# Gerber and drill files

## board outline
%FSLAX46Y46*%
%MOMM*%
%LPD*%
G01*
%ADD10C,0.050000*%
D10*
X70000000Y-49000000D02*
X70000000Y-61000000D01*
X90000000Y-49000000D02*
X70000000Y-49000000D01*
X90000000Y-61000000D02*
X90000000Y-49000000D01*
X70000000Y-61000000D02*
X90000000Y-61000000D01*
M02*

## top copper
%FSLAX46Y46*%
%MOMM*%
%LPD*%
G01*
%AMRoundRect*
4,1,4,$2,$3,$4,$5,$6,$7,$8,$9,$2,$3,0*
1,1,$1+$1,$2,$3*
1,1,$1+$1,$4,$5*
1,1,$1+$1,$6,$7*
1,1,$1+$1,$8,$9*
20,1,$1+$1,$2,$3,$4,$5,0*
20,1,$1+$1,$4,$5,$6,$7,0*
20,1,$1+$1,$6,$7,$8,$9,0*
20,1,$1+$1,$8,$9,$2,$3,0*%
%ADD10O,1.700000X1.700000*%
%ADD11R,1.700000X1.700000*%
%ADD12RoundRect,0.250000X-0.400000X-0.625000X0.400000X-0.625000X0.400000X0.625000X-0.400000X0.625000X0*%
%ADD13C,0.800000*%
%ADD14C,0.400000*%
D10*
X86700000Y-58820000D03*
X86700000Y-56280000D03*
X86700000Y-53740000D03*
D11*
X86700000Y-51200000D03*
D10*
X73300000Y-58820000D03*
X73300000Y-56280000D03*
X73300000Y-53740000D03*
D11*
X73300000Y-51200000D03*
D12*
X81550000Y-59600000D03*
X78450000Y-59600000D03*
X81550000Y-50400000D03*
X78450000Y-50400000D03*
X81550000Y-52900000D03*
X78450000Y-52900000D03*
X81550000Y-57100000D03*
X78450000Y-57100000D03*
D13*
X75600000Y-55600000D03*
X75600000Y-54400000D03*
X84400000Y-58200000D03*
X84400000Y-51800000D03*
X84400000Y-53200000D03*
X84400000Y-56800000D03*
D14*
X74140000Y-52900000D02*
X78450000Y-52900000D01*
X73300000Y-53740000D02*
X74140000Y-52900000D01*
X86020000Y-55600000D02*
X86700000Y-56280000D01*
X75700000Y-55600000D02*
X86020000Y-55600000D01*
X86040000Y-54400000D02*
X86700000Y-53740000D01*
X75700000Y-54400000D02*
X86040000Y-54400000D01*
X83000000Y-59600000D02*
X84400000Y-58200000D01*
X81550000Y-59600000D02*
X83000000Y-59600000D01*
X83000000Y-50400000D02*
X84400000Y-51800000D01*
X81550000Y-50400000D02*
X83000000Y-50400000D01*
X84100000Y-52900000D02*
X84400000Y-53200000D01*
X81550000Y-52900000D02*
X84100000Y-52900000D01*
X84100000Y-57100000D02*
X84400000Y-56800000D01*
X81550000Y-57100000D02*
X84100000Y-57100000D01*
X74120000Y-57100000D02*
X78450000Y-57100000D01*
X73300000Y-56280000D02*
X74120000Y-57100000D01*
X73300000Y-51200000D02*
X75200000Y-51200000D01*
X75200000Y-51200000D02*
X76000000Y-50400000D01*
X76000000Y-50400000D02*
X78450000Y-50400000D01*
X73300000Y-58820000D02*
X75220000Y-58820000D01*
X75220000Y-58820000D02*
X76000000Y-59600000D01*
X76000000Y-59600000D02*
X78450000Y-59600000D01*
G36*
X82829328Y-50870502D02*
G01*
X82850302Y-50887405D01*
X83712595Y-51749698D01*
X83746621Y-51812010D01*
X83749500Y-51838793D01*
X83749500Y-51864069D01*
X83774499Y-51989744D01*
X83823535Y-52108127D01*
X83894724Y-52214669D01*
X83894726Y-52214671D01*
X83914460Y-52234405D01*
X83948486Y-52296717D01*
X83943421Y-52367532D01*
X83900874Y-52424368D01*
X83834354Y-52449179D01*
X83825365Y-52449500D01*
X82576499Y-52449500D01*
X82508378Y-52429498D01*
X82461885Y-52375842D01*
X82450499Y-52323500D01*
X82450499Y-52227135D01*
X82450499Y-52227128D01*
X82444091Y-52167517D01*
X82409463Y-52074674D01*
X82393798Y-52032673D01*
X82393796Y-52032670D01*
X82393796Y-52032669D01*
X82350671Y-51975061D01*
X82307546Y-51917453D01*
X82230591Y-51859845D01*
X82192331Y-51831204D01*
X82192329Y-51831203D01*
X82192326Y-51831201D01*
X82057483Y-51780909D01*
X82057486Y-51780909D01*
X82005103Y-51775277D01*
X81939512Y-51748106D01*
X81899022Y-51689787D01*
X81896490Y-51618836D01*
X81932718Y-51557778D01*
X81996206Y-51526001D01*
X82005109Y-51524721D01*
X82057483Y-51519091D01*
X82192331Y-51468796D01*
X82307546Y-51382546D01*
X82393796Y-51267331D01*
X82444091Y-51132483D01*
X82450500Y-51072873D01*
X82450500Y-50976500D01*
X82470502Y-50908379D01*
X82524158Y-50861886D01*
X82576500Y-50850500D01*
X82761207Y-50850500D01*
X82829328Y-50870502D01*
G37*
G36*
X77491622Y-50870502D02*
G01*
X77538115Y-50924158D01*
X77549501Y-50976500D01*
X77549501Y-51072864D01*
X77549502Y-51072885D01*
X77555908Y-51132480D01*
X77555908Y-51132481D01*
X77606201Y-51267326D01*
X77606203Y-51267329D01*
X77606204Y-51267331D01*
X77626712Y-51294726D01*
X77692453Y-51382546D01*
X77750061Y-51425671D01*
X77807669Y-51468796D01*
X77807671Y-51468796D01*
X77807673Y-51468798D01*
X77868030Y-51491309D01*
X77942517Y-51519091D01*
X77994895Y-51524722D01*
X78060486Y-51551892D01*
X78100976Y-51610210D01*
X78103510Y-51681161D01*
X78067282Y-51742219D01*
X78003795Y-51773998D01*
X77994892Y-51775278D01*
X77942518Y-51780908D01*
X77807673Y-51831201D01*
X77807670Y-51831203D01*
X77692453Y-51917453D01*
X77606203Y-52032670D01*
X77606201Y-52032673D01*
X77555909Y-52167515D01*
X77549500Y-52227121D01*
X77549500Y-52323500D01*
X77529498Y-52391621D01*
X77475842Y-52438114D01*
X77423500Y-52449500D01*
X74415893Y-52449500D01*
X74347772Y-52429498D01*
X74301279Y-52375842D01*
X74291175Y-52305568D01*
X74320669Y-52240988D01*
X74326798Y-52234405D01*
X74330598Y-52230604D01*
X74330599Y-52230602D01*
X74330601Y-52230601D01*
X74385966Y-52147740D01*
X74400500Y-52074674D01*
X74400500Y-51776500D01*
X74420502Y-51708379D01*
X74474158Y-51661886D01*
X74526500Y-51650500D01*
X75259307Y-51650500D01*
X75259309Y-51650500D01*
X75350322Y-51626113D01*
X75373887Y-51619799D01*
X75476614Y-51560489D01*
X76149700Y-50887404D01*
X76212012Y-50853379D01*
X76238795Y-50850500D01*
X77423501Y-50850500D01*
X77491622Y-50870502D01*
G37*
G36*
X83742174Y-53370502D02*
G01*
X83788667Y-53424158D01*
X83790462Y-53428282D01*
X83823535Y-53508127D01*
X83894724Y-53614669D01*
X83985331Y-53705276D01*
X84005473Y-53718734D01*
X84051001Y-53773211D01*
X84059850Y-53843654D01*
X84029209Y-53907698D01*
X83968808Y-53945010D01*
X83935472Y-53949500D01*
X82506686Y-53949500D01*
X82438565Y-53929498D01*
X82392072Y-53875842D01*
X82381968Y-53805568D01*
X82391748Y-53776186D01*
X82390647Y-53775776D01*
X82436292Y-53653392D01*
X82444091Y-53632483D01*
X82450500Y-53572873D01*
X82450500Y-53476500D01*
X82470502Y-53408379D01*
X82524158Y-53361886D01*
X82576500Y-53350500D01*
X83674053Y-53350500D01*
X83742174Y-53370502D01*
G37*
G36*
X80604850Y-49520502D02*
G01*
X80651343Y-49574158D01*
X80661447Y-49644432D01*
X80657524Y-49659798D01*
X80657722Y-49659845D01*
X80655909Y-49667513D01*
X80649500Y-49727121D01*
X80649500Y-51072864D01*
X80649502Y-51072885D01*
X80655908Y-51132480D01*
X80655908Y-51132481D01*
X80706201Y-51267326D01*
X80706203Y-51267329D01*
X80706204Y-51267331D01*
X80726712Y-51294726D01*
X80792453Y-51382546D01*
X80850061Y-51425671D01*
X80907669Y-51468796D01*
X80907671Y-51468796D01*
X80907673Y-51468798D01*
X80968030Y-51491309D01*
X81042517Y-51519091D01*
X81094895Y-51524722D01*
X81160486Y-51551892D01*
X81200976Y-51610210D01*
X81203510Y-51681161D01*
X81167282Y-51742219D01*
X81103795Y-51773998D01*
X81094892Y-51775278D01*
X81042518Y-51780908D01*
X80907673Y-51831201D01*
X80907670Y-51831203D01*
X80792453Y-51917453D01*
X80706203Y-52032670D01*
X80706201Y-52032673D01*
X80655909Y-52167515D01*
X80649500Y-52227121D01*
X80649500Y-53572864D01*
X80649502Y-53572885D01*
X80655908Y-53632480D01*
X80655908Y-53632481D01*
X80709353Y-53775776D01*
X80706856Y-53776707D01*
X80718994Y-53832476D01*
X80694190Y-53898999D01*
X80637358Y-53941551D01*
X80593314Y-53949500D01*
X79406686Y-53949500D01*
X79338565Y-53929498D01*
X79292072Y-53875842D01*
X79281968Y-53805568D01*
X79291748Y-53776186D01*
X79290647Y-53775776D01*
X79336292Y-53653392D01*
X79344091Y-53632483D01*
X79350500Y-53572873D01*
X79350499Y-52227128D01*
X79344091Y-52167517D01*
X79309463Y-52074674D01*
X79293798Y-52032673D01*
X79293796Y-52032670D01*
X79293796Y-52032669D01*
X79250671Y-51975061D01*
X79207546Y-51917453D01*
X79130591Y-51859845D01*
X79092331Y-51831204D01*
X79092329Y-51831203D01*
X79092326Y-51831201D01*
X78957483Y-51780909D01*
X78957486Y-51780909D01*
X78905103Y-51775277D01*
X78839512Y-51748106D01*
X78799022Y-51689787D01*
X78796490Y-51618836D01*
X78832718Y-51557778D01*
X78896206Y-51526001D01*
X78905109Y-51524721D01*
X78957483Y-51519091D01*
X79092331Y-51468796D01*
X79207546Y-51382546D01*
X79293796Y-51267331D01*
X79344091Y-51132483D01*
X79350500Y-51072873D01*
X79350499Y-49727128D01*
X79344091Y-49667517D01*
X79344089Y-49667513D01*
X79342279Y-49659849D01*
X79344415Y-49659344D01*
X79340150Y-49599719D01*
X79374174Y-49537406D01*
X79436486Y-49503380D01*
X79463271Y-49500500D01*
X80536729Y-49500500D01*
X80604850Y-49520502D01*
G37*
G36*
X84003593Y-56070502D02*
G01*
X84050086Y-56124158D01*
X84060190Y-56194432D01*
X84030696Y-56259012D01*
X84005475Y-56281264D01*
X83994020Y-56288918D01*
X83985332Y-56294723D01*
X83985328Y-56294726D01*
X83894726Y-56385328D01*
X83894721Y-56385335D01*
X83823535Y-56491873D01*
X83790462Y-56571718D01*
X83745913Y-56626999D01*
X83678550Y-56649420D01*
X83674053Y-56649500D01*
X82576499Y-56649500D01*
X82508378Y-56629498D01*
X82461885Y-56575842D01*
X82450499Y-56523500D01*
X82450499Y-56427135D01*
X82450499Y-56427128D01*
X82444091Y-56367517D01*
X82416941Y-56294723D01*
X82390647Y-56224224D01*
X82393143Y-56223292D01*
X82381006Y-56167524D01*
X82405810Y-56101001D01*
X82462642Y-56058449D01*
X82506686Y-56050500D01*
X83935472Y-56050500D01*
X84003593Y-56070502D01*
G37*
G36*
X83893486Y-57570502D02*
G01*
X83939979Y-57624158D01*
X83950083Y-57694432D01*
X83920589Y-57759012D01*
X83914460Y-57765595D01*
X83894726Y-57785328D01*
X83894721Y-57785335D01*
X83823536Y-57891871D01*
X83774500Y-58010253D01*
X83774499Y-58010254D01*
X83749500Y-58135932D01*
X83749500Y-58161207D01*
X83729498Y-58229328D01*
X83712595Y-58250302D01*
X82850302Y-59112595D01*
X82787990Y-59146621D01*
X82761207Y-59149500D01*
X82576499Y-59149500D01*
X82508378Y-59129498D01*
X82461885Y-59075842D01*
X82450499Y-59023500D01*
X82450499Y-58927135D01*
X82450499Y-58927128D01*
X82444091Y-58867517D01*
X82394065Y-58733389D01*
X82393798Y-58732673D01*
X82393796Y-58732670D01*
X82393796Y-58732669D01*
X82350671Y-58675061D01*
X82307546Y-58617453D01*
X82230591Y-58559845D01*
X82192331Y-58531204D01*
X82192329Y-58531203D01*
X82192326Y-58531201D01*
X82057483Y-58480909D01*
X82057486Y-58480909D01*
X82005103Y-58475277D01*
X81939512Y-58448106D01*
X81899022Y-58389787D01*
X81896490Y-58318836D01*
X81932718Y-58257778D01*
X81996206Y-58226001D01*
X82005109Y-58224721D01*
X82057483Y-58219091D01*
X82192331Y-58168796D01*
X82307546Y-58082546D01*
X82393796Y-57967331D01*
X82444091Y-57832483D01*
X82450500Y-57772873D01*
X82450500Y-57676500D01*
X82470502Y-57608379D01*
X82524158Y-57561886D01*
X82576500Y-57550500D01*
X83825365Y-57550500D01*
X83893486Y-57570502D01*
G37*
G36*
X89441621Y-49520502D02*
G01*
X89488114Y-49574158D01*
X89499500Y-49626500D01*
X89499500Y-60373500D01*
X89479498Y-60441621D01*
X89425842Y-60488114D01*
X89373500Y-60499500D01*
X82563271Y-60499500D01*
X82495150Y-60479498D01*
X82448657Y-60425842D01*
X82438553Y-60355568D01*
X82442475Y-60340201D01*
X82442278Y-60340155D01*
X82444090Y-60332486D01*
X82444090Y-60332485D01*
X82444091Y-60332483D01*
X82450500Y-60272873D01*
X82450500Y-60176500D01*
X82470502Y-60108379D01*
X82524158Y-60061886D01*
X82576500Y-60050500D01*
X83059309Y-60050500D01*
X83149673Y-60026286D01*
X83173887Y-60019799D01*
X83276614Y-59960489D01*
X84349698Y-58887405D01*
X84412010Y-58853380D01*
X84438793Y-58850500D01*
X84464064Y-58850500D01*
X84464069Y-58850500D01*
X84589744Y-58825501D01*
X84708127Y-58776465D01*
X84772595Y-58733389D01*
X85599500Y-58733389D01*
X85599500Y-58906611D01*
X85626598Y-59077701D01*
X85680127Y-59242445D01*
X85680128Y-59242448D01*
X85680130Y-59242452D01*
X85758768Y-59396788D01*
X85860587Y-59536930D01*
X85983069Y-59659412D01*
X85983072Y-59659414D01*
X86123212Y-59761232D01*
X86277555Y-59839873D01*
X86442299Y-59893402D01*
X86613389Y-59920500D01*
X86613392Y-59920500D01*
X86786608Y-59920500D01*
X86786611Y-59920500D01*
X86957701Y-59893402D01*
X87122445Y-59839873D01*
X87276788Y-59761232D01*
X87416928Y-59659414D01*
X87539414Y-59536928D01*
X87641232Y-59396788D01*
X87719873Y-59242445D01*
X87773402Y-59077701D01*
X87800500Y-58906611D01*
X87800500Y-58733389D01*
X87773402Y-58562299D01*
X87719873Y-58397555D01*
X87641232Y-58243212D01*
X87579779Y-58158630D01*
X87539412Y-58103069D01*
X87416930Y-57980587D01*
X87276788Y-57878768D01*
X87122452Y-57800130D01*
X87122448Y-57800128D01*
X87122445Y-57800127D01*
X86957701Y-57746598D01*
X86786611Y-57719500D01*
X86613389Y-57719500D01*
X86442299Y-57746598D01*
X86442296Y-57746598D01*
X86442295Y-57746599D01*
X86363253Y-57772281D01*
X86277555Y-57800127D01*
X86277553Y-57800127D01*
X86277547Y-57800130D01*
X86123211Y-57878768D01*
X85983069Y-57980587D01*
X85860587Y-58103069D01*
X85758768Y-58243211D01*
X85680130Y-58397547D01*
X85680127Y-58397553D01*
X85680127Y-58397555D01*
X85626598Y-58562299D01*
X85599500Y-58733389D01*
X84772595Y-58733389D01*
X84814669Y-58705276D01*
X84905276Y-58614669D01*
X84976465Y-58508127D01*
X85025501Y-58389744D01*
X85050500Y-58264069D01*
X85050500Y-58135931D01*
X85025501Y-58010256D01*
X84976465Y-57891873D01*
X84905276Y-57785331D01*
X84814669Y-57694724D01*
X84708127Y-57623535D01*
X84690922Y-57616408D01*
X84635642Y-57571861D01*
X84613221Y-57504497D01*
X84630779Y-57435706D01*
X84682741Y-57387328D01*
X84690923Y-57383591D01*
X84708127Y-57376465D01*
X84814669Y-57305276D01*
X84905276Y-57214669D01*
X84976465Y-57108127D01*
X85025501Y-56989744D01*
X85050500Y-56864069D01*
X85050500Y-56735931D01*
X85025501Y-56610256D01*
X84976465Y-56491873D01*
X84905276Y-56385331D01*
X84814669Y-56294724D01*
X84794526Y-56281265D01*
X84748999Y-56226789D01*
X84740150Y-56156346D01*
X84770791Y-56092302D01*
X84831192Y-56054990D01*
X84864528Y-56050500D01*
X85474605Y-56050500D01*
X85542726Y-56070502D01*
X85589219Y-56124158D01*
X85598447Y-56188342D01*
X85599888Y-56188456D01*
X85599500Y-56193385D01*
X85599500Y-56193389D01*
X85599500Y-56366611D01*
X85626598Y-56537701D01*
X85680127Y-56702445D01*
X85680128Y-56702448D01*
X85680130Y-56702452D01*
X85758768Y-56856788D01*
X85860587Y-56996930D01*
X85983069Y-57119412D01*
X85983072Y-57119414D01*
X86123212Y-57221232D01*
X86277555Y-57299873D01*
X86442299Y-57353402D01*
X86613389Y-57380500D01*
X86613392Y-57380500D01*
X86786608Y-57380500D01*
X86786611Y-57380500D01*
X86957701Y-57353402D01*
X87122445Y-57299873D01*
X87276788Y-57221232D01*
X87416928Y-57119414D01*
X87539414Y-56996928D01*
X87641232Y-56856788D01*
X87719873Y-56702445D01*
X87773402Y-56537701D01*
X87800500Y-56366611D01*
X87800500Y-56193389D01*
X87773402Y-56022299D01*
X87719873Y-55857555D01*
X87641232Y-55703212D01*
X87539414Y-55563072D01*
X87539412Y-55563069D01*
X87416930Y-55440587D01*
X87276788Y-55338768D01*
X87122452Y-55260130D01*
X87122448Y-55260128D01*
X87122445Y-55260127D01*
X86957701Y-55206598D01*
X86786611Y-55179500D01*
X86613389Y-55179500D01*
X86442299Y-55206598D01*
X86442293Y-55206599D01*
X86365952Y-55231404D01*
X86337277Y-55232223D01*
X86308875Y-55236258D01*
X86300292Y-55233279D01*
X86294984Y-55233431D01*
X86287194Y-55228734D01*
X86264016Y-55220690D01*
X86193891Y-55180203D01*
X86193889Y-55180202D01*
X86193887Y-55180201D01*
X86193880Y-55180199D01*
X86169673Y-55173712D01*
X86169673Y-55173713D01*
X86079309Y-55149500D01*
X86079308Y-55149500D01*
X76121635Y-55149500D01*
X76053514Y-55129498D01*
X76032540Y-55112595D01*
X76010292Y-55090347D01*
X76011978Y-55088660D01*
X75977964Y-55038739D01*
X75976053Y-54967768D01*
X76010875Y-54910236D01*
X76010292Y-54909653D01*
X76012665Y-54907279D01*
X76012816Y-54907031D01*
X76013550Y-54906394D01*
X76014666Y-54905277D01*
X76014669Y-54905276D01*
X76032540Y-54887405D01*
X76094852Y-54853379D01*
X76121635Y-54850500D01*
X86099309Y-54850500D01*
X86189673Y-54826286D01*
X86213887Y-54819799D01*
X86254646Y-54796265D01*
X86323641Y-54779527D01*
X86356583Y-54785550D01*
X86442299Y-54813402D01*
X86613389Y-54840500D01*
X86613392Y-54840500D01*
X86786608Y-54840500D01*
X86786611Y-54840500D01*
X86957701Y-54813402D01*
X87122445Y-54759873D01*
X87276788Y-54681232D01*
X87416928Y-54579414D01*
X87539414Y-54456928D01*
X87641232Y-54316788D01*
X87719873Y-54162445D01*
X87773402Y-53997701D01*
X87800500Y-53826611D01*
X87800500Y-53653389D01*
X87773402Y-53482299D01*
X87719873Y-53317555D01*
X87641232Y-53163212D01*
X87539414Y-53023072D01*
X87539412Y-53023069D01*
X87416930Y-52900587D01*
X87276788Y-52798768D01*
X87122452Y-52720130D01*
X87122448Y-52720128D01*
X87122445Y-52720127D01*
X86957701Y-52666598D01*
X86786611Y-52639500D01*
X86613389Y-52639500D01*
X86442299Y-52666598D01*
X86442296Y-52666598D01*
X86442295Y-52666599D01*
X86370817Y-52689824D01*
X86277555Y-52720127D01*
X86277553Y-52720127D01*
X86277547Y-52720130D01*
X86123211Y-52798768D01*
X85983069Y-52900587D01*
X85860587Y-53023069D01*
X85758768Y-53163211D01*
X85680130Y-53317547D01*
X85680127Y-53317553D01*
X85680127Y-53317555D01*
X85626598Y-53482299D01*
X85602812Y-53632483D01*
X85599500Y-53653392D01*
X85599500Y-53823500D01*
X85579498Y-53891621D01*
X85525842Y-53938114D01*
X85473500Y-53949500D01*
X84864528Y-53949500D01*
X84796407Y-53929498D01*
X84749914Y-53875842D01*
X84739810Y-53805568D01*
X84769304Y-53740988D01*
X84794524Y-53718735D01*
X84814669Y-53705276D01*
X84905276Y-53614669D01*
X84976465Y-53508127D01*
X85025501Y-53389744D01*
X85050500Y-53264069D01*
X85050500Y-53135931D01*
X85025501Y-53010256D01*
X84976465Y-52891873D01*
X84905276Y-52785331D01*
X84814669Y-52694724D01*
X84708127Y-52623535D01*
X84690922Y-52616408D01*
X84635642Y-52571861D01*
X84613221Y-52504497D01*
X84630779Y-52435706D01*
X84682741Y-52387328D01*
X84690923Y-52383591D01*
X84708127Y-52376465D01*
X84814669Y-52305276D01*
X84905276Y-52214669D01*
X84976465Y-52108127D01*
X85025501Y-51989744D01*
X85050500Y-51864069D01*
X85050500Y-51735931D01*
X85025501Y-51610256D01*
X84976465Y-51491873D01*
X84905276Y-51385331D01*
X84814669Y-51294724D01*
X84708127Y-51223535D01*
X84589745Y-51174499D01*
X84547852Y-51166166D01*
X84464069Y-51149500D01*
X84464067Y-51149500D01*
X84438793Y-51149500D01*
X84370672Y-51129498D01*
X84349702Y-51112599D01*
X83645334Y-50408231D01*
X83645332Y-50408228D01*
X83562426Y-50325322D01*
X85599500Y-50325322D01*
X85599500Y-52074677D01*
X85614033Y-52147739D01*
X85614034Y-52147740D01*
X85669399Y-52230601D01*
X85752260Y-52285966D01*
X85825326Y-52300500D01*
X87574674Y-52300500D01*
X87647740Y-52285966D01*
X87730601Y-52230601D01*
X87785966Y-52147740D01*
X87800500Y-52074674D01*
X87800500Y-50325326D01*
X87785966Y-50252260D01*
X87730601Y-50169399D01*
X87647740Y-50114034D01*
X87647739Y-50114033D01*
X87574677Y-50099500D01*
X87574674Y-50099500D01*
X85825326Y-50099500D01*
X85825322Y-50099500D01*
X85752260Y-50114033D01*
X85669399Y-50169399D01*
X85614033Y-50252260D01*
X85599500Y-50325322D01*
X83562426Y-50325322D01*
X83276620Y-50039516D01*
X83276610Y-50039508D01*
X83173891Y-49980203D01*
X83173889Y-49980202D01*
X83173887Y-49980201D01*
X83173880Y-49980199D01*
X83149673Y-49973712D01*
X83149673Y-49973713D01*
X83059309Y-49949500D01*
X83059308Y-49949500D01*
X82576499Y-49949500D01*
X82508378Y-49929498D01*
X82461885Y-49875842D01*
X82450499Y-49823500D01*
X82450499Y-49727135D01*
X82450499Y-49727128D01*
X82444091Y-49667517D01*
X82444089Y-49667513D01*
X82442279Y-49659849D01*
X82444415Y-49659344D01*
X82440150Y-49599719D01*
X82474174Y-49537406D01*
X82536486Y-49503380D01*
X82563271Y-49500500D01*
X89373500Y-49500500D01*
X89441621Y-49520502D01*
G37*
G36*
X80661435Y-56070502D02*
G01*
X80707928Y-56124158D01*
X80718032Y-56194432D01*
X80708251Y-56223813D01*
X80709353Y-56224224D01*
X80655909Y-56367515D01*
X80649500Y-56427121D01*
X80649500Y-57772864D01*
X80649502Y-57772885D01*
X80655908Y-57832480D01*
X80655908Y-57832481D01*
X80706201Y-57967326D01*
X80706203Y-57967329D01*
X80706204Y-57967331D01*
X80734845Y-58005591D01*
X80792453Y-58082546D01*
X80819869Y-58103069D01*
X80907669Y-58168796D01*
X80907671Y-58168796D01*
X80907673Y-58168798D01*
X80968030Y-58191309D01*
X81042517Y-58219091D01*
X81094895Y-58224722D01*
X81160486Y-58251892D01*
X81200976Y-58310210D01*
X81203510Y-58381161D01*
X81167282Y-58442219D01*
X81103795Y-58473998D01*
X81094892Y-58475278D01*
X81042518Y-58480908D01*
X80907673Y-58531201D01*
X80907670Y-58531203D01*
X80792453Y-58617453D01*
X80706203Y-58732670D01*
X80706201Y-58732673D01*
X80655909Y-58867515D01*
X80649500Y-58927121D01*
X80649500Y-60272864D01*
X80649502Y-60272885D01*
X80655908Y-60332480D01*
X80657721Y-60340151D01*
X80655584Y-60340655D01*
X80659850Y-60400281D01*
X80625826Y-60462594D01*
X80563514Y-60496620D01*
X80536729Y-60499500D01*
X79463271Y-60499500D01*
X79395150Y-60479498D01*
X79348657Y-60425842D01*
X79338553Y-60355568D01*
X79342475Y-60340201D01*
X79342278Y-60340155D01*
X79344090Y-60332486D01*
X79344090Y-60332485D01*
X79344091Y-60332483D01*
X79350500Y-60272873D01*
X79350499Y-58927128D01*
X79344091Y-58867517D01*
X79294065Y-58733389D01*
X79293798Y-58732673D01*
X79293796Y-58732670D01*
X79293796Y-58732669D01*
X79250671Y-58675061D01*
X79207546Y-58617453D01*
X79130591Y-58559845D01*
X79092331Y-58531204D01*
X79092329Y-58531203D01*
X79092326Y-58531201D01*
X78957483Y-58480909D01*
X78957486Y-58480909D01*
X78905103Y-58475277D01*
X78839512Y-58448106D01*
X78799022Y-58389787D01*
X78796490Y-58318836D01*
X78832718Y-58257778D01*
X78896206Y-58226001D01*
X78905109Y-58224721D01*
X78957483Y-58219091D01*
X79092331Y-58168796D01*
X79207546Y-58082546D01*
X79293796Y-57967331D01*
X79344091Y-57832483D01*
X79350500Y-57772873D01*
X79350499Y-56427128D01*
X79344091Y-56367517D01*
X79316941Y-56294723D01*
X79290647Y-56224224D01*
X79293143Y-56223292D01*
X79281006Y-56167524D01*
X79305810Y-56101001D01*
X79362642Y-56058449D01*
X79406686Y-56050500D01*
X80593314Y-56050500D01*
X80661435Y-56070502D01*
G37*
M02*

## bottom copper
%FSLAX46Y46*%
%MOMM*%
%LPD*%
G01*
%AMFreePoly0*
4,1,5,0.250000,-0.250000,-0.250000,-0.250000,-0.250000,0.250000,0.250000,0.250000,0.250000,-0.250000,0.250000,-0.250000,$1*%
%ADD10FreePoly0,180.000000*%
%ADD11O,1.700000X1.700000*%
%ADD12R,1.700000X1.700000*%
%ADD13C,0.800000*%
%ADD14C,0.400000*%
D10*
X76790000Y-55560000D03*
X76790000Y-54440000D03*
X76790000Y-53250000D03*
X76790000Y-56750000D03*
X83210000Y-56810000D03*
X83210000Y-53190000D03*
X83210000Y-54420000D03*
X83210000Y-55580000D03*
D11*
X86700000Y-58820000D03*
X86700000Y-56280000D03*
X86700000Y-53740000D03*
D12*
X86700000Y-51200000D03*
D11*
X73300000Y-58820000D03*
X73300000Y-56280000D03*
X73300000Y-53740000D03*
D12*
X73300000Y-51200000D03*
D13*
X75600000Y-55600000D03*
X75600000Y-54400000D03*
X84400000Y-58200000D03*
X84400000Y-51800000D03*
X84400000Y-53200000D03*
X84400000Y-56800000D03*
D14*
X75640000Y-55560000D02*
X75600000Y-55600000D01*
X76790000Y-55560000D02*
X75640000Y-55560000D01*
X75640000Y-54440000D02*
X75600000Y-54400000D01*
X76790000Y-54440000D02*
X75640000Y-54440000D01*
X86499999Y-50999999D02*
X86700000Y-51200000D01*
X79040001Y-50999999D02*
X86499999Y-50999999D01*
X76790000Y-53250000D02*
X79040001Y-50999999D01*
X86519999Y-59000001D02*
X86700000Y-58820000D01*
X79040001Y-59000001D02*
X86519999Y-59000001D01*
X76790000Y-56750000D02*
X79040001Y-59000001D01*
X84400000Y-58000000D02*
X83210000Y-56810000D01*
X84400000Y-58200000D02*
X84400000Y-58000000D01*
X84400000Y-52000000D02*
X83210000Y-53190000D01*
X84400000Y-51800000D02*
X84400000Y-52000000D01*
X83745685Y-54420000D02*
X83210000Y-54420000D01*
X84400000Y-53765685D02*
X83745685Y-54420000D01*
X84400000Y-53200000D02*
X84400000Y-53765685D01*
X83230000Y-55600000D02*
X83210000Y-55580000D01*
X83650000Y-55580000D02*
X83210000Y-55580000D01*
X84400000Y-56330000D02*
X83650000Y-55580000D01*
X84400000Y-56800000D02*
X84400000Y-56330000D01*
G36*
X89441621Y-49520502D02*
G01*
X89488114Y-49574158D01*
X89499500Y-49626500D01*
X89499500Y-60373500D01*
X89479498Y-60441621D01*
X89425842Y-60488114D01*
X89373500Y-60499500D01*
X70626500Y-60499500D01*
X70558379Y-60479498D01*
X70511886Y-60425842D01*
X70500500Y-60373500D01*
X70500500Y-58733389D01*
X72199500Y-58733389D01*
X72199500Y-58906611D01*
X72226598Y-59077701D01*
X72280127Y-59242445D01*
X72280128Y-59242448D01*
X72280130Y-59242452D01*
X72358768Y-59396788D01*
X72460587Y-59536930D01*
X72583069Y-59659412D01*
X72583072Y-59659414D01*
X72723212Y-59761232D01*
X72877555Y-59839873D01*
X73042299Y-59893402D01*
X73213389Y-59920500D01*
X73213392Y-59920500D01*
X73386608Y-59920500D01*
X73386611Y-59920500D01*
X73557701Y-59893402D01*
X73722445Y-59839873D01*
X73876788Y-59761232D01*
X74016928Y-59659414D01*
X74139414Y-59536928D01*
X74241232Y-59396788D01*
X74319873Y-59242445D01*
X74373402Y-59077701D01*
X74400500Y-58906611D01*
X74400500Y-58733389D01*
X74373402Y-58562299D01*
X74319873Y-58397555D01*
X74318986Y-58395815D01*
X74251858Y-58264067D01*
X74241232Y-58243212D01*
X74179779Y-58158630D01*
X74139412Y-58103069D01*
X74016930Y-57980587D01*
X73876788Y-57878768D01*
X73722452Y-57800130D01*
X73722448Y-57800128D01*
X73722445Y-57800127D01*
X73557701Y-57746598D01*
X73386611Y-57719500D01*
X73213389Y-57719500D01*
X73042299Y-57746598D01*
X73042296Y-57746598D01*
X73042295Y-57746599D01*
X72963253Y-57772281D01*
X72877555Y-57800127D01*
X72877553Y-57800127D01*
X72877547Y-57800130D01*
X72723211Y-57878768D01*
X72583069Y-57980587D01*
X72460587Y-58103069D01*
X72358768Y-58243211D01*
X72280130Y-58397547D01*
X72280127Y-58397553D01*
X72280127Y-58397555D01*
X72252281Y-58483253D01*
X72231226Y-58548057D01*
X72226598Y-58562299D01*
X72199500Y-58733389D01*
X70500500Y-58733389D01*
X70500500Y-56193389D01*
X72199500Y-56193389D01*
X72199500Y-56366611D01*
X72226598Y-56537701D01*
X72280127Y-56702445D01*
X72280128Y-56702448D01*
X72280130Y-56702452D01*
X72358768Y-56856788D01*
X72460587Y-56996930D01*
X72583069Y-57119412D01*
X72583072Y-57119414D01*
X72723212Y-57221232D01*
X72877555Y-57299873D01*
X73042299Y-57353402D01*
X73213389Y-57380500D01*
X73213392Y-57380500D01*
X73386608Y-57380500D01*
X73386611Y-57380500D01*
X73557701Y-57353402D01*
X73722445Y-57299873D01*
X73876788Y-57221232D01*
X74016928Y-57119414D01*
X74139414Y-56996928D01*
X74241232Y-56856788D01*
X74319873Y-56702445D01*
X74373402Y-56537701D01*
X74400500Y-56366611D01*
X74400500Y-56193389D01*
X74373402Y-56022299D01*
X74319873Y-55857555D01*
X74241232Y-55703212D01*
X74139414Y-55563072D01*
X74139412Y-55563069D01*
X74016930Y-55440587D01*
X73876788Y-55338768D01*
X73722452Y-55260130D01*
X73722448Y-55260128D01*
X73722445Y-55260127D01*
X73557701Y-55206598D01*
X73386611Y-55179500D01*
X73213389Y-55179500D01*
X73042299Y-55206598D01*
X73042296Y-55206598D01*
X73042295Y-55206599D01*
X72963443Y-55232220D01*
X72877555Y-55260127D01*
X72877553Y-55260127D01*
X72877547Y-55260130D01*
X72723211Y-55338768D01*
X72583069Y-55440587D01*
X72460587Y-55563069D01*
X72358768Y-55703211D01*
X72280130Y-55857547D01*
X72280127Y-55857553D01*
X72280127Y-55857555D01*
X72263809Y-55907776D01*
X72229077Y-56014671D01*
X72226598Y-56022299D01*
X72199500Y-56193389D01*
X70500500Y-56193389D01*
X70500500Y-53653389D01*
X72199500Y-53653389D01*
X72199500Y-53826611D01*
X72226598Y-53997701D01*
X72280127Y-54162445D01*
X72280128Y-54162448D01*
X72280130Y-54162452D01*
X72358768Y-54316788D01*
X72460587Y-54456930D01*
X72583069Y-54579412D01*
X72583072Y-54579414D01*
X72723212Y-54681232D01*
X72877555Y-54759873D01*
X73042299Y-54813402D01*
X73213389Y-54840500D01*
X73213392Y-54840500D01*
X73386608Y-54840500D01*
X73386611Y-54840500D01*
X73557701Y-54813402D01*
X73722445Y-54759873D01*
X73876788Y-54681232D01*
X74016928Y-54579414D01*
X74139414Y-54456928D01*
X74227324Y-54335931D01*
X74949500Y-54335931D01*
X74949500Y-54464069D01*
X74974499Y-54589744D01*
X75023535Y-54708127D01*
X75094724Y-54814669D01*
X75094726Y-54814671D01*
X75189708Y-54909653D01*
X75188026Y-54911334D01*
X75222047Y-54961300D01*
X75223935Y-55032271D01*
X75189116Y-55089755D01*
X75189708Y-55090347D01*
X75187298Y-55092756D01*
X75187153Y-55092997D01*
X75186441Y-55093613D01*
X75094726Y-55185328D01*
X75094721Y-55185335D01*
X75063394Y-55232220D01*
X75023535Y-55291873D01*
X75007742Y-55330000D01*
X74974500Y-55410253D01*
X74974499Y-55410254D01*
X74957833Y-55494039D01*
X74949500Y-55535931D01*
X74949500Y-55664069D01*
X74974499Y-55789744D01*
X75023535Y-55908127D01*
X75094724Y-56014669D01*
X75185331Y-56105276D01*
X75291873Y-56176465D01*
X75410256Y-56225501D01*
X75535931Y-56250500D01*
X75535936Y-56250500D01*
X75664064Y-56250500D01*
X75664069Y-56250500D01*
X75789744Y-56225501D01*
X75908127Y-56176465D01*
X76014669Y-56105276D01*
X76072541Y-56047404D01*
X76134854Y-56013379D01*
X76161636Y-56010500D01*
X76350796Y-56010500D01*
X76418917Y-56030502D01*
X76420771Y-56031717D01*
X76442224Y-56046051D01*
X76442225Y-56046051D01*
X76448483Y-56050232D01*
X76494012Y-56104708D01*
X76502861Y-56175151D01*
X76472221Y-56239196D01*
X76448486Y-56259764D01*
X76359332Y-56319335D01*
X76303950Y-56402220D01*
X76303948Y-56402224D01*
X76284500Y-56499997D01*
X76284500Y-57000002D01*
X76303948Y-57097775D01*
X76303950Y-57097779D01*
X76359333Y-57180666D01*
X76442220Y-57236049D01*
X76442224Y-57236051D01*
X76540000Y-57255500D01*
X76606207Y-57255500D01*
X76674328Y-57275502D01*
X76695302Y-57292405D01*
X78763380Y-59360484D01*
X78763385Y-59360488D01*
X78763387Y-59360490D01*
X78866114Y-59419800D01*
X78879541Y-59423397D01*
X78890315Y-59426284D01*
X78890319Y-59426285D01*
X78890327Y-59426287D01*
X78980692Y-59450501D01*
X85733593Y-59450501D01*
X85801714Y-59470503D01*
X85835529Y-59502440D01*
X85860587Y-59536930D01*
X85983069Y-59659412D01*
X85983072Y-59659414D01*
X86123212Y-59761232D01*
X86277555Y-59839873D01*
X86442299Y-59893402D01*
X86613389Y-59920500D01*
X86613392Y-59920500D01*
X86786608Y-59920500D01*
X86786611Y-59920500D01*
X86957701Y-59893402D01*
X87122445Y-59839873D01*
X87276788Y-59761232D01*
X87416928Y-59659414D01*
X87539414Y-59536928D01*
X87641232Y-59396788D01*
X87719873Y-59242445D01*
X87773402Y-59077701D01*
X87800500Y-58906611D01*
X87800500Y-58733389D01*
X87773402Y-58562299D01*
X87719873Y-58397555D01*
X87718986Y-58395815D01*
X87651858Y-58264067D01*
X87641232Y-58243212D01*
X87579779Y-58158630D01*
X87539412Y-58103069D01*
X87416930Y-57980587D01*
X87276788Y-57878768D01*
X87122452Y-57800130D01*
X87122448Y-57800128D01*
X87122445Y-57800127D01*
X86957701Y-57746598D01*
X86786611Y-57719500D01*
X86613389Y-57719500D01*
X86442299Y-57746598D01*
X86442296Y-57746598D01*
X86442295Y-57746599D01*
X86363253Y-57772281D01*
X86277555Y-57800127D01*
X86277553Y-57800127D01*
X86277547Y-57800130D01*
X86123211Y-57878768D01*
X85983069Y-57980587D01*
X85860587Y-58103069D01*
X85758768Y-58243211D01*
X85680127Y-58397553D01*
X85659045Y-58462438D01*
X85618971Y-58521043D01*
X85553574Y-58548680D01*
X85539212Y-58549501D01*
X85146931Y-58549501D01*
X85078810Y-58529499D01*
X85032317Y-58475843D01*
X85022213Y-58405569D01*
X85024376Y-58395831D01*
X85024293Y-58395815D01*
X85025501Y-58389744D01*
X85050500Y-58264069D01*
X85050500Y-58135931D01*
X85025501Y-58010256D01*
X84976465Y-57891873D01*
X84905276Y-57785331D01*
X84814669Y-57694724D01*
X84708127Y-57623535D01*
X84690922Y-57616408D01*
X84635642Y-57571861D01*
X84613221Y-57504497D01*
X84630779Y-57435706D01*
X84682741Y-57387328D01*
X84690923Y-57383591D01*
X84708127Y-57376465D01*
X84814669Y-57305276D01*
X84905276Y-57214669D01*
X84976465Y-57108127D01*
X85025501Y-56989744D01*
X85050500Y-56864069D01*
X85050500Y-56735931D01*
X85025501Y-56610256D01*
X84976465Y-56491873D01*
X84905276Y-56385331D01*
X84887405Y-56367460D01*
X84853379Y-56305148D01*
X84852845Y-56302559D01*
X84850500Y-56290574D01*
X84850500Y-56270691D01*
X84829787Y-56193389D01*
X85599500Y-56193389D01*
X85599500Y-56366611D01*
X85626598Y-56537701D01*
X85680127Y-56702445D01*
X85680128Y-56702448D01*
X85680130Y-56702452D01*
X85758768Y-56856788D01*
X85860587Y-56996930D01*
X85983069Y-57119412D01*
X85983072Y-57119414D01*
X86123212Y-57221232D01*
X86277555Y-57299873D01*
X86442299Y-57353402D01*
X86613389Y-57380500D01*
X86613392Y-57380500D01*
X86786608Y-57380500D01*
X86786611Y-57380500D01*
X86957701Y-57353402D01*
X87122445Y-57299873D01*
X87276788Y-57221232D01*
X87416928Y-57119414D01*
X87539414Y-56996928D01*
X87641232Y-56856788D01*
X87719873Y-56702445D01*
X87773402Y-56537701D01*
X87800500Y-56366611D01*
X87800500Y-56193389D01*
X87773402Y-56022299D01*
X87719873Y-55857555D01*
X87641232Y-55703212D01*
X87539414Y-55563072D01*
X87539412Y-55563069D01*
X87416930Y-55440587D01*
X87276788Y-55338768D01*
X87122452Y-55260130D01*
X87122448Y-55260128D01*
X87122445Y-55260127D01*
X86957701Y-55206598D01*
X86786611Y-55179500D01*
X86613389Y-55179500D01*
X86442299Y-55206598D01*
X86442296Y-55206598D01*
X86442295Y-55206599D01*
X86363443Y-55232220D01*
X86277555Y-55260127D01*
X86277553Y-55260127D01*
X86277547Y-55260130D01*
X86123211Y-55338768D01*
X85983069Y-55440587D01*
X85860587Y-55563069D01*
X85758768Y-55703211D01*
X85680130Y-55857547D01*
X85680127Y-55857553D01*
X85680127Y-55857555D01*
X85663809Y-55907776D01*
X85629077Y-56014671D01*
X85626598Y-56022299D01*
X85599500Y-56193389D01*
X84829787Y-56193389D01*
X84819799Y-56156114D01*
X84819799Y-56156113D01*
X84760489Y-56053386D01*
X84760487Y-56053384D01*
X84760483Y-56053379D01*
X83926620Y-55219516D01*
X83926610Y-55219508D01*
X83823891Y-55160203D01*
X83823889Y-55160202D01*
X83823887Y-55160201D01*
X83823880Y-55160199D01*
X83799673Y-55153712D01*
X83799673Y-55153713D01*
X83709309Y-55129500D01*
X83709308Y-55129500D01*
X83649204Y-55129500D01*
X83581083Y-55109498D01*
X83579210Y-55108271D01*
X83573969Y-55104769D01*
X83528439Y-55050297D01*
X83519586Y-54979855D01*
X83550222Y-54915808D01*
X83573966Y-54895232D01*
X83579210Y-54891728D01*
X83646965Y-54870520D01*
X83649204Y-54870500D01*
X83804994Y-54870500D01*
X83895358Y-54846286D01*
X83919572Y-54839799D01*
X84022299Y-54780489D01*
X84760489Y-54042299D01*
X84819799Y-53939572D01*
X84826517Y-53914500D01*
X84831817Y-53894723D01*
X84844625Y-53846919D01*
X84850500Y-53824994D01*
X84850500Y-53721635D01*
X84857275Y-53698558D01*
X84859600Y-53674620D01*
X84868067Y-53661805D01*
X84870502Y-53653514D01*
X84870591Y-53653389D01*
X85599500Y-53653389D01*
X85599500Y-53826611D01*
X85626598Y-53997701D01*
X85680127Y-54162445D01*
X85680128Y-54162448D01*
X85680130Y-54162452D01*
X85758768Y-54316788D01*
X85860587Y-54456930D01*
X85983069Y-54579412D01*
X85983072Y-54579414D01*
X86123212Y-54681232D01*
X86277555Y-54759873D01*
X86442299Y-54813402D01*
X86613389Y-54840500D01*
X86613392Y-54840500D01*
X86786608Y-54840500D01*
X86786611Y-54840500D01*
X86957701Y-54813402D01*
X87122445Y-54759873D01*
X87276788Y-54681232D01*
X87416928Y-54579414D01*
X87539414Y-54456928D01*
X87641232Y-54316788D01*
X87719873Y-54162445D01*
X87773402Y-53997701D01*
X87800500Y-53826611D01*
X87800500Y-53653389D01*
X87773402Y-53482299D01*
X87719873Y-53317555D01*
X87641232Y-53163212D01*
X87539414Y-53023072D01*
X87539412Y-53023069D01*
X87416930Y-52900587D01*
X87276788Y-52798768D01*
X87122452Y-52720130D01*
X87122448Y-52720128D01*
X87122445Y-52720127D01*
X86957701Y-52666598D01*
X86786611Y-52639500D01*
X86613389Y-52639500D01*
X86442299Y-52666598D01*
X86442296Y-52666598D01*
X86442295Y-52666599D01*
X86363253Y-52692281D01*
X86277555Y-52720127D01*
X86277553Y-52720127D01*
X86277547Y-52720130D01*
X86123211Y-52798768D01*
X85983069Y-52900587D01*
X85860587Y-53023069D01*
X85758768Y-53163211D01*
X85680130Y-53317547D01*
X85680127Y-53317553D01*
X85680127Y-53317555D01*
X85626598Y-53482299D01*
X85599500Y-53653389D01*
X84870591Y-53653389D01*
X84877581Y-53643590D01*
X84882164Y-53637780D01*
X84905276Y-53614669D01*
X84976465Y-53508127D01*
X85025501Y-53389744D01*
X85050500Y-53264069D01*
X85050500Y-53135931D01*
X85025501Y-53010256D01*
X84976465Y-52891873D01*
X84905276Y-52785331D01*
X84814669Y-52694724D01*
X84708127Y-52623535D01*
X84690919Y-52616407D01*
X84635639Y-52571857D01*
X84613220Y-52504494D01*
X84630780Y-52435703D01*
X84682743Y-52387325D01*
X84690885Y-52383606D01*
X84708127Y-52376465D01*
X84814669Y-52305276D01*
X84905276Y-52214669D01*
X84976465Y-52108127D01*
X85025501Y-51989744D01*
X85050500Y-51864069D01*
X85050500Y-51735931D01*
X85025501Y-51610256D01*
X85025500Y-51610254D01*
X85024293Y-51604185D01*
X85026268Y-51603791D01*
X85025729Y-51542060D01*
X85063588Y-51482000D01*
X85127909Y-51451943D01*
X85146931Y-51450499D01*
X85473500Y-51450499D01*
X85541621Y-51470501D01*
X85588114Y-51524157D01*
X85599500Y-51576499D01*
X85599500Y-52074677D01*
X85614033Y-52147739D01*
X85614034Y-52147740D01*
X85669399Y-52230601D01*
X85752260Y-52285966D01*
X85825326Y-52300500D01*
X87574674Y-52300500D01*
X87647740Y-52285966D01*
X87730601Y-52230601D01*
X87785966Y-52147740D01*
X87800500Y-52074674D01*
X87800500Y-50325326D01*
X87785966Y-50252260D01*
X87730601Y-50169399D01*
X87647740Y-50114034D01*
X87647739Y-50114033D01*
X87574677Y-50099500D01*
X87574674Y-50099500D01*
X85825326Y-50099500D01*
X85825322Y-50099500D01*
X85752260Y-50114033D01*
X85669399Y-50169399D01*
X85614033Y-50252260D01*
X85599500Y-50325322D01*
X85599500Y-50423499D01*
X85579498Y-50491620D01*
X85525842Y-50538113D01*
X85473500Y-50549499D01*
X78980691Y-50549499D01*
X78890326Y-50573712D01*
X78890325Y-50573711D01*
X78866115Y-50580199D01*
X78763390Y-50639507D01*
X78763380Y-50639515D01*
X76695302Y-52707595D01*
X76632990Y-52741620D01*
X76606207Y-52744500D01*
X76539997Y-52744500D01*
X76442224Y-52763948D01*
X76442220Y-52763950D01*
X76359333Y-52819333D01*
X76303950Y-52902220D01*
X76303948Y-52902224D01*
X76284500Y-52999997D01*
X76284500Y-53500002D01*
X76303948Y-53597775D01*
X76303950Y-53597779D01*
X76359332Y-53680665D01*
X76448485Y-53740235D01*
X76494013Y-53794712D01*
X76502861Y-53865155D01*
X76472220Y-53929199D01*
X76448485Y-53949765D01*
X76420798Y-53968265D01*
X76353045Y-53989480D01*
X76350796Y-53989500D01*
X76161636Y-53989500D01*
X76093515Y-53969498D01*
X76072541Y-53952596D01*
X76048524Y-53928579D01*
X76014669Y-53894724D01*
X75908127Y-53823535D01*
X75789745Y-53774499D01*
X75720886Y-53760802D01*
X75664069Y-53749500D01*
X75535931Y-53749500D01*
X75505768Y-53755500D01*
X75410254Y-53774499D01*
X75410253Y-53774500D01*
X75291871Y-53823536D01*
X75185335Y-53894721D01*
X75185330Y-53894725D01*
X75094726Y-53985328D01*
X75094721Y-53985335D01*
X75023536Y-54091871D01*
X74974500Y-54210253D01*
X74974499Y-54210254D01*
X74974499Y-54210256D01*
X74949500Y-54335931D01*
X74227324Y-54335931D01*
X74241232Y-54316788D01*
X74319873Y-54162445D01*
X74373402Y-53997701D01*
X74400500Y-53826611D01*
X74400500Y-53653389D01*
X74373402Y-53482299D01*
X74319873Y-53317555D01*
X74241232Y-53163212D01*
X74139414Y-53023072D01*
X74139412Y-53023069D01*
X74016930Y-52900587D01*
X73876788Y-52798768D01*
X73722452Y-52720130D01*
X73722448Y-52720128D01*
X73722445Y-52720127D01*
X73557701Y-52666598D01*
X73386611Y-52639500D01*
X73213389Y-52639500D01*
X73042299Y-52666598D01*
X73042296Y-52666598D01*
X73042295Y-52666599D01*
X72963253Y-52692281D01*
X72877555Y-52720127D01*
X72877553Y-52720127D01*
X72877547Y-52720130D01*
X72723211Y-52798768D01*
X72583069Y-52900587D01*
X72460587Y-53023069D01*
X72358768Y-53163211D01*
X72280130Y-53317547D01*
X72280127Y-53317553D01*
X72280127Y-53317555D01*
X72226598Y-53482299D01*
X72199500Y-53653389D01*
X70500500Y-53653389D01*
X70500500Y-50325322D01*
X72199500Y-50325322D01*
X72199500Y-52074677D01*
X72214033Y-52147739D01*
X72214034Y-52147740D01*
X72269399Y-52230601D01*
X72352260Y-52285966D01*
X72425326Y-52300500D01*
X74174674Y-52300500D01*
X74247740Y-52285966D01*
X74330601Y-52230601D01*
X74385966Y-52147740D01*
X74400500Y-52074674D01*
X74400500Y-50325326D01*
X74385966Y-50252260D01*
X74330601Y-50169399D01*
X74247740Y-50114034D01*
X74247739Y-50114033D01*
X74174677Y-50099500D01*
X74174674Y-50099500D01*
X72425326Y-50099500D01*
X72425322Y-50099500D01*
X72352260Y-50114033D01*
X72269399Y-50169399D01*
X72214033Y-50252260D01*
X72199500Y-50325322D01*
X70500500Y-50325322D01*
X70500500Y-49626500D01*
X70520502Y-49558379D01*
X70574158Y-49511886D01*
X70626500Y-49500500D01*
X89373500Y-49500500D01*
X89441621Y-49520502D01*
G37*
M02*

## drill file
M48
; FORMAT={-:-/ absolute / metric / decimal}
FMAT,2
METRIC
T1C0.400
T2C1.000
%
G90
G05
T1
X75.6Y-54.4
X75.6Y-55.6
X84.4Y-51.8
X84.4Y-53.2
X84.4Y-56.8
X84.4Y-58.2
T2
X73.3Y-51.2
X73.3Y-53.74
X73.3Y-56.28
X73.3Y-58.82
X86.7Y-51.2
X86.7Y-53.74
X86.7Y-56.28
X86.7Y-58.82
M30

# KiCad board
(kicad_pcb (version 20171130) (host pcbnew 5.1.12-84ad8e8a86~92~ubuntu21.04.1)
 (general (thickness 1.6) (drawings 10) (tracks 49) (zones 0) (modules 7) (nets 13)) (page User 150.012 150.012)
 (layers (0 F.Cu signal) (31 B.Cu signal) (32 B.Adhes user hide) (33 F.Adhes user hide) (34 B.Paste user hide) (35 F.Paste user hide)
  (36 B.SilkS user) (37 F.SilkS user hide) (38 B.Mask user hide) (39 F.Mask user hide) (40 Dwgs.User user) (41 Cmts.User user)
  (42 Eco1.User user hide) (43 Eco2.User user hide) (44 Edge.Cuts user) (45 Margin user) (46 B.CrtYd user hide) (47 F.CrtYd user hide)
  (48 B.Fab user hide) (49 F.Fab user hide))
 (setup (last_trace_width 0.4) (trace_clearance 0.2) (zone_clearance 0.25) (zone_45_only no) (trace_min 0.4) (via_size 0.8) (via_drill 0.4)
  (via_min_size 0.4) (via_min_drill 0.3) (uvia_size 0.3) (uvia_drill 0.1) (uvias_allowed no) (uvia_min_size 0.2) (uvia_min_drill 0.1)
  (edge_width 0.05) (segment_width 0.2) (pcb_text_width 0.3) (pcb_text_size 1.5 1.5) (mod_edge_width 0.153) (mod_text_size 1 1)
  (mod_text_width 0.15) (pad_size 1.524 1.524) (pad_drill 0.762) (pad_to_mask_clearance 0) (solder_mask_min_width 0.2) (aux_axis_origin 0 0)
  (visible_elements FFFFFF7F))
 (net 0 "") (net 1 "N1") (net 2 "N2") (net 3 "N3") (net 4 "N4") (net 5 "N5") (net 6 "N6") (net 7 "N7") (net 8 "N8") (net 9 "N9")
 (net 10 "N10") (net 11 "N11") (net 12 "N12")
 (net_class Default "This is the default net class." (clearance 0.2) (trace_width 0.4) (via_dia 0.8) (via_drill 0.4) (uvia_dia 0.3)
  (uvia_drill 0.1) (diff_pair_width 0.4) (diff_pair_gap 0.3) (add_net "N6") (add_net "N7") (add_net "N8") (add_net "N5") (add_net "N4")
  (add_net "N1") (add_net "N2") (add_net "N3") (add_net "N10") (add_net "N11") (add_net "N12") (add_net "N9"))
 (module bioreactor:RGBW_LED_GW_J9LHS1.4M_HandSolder (layer B.Cu) (at 80 55 180)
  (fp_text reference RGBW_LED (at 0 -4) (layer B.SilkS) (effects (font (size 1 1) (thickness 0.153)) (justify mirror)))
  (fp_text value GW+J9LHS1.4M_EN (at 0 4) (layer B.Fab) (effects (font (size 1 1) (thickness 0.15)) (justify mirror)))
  (pad 6 smd custom (at 3.21 -0.56 180) (size 0.5 0.5) (layers B.Cu B.Paste B.Mask) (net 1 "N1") (zone_connect 0)
   (options (clearance outline) (anchor rect)) (primitives))
  (pad 7 smd custom (at 3.21 0.56 180) (size 0.5 0.5) (layers B.Cu B.Paste B.Mask) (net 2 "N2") (zone_connect 0)
   (options (clearance outline) (anchor rect)) (primitives))
  (pad 8 smd custom (at 3.21 1.75 180) (size 0.5 0.5) (layers B.Cu B.Paste B.Mask) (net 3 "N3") (zone_connect 0)
   (options (clearance outline) (anchor rect)) (primitives))
  (pad 5 smd custom (at 3.21 -1.75 180) (size 0.5 0.5) (layers B.Cu B.Paste B.Mask) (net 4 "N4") (zone_connect 0)
   (options (clearance outline) (anchor rect)) (primitives))
  (pad 4 smd custom (at -3.21 -1.81 180) (size 0.5 0.5) (layers B.Cu B.Paste B.Mask) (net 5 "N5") (zone_connect 0)
   (options (clearance outline) (anchor rect)) (primitives))
  (pad 1 smd custom (at -3.21 1.81 180) (size 0.5 0.5) (layers B.Cu B.Paste B.Mask) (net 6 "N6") (zone_connect 0)
   (options (clearance outline) (anchor rect)) (primitives))
  (pad 2 smd custom (at -3.21 0.58 180) (size 0.5 0.5) (layers B.Cu B.Paste B.Mask) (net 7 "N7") (zone_connect 0)
   (options (clearance outline) (anchor rect)) (primitives))
  (pad 3 smd custom (at -3.21 -0.58 180) (size 0.5 0.5) (layers B.Cu B.Paste B.Mask) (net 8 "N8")
   (options (clearance outline) (anchor rect)) (primitives)))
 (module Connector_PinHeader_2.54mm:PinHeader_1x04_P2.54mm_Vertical (layer F.Cu) (at 86.7 51.2)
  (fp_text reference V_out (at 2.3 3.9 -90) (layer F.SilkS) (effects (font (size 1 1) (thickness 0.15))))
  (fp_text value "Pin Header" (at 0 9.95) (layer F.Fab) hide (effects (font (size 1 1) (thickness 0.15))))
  (pad 4 thru_hole oval (at 0 7.62) (size 1.7 1.7) (drill 1) (layers *.Cu *.Mask) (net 4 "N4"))
  (pad 3 thru_hole oval (at 0 5.08) (size 1.7 1.7) (drill 1) (layers *.Cu *.Mask) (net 1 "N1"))
  (pad 2 thru_hole oval (at 0 2.54) (size 1.7 1.7) (drill 1) (layers *.Cu *.Mask) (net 2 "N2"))
  (pad 1 thru_hole rect (at 0 0) (size 1.7 1.7) (drill 1) (layers *.Cu *.Mask) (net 3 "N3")))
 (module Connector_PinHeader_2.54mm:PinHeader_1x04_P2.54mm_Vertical (layer F.Cu) (at 73.3 51.2)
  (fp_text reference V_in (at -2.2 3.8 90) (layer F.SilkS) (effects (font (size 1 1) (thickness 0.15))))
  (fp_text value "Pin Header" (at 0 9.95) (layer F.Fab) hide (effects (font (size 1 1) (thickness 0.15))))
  (pad 4 thru_hole oval (at 0 7.62) (size 1.7 1.7) (drill 1) (layers *.Cu *.Mask) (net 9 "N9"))
  (pad 3 thru_hole oval (at 0 5.08) (size 1.7 1.7) (drill 1) (layers *.Cu *.Mask) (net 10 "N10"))
  (pad 2 thru_hole oval (at 0 2.54) (size 1.7 1.7) (drill 1) (layers *.Cu *.Mask) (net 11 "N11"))
  (pad 1 thru_hole rect (at 0 0) (size 1.7 1.7) (drill 1) (layers *.Cu *.Mask) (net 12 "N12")))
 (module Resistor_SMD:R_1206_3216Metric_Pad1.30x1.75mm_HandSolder (layer F.Cu) (at 80 59.6)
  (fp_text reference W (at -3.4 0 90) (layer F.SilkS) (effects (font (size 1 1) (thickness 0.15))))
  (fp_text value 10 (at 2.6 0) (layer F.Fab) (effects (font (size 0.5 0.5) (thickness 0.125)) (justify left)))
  (pad 2 smd roundrect (at 1.55 0) (size 1.3 1.75) (layers F.Cu F.Paste F.Mask) (roundrect_rratio 0.1923076923076923) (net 5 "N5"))
  (pad 1 smd roundrect (at -1.55 0) (size 1.3 1.75) (layers F.Cu F.Paste F.Mask) (roundrect_rratio 0.1923076923076923) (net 9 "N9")))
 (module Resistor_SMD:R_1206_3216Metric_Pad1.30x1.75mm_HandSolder (layer F.Cu) (at 80 50.4)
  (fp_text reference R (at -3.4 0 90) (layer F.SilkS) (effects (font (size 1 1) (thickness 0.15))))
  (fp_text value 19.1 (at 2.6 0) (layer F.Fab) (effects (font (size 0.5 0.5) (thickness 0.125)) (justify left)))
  (pad 2 smd roundrect (at 1.55 0) (size 1.3 1.75) (layers F.Cu F.Paste F.Mask) (roundrect_rratio 0.1923076923076923) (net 6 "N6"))
  (pad 1 smd roundrect (at -1.55 0) (size 1.3 1.75) (layers F.Cu F.Paste F.Mask) (roundrect_rratio 0.1923076923076923) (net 12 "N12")))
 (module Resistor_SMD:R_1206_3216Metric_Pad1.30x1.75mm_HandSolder (layer F.Cu) (at 80 52.9)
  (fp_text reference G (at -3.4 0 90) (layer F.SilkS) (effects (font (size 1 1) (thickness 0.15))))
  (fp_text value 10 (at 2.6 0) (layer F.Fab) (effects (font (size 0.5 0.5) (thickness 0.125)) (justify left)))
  (pad 2 smd roundrect (at 1.55 0) (size 1.3 1.75) (layers F.Cu F.Paste F.Mask) (roundrect_rratio 0.1923076923076923) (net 7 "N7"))
  (pad 1 smd roundrect (at -1.55 0) (size 1.3 1.75) (layers F.Cu F.Paste F.Mask) (roundrect_rratio 0.1923076923076923) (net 11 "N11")))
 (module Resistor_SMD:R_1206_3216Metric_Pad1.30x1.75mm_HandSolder (layer F.Cu) (at 80 57.1)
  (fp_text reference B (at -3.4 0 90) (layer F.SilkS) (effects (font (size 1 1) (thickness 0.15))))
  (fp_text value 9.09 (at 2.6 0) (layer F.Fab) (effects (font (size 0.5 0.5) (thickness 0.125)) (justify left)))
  (pad 2 smd roundrect (at 1.55 0) (size 1.3 1.75) (layers F.Cu F.Paste F.Mask) (roundrect_rratio 0.1923076923076923) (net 8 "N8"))
  (pad 1 smd roundrect (at -1.55 0) (size 1.3 1.75) (layers F.Cu F.Paste F.Mask) (roundrect_rratio 0.1923076923076923) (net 10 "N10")))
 (gr_line (start 70 49) (end 70 61) (layer Edge.Cuts) (width 0.05))
 (gr_line (start 90 49) (end 70 49) (layer Edge.Cuts) (width 0.05))
 (gr_line (start 90 61) (end 90 49) (layer Edge.Cuts) (width 0.05))
 (gr_line (start 70 61) (end 90 61) (layer Edge.Cuts) (width 0.05))
 (segment (start 74.14 52.9) (end 78.45 52.9) (width 0.4) (layer F.Cu) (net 11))
 (segment (start 73.3 53.74) (end 74.14 52.9) (width 0.4) (layer F.Cu) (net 11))
 (via (at 75.6 55.6) (size 0.8) (drill 0.4) (layers F.Cu B.Cu) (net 1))
 (segment (start 86.02 55.6) (end 86.7 56.28) (width 0.4) (layer F.Cu) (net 1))
 (segment (start 75.7 55.6) (end 86.02 55.6) (width 0.4) (layer F.Cu) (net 1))
 (segment (start 75.64 55.56) (end 75.6 55.6) (width 0.4) (layer B.Cu) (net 1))
 (segment (start 76.79 55.56) (end 75.64 55.56) (width 0.4) (layer B.Cu) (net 1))
 (via (at 75.6 54.4) (size 0.8) (drill 0.4) (layers F.Cu B.Cu) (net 2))
 (segment (start 86.04 54.4) (end 86.7 53.74) (width 0.4) (layer F.Cu) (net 2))
 (segment (start 75.7 54.4) (end 86.04 54.4) (width 0.4) (layer F.Cu) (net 2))
 (segment (start 75.64 54.44) (end 75.6 54.4) (width 0.4) (layer B.Cu) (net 2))
 (segment (start 76.79 54.44) (end 75.64 54.44) (width 0.4) (layer B.Cu) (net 2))
 (segment (start 86.499999 50.999999) (end 86.7 51.2) (width 0.4) (layer B.Cu) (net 3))
 (segment (start 79.040001 50.999999) (end 86.499999 50.999999) (width 0.4) (layer B.Cu) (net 3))
 (segment (start 76.79 53.25) (end 79.040001 50.999999) (width 0.4) (layer B.Cu) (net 3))
 (segment (start 86.519999 59.000001) (end 86.7 58.82) (width 0.4) (layer B.Cu) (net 4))
 (segment (start 79.040001 59.000001) (end 86.519999 59.000001) (width 0.4) (layer B.Cu) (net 4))
 (segment (start 76.79 56.75) (end 79.040001 59.000001) (width 0.4) (layer B.Cu) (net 4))
 (via (at 84.4 58.2) (size 0.8) (drill 0.4) (layers F.Cu B.Cu) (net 5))
 (segment (start 84.4 58) (end 83.21 56.81) (width 0.4) (layer B.Cu) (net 5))
 (segment (start 84.4 58.2) (end 84.4 58) (width 0.4) (layer B.Cu) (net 5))
 (segment (start 83 59.6) (end 84.4 58.2) (width 0.4) (layer F.Cu) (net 5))
 (segment (start 81.55 59.6) (end 83 59.6) (width 0.4) (layer F.Cu) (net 5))
 (via (at 84.4 51.8) (size 0.8) (drill 0.4) (layers F.Cu B.Cu) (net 6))
 (segment (start 84.4 52) (end 83.21 53.19) (width 0.4) (layer B.Cu) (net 6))
 (segment (start 84.4 51.8) (end 84.4 52) (width 0.4) (layer B.Cu) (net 6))
 (segment (start 83 50.4) (end 84.4 51.8) (width 0.4) (layer F.Cu) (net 6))
 (segment (start 81.55 50.4) (end 83 50.4) (width 0.4) (layer F.Cu) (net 6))
 (via (at 84.4 53.2) (size 0.8) (drill 0.4) (layers F.Cu B.Cu) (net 7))
 (segment (start 83.745685 54.42) (end 83.21 54.42) (width 0.4) (layer B.Cu) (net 7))
 (segment (start 84.4 53.765685) (end 83.745685 54.42) (width 0.4) (layer B.Cu) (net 7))
 (segment (start 84.4 53.2) (end 84.4 53.765685) (width 0.4) (layer B.Cu) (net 7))
 (segment (start 84.1 52.9) (end 84.4 53.2) (width 0.4) (layer F.Cu) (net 7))
 (segment (start 81.55 52.9) (end 84.1 52.9) (width 0.4) (layer F.Cu) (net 7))
 (via (at 84.4 56.8) (size 0.8) (drill 0.4) (layers F.Cu B.Cu) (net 8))
 (segment (start 83.23 55.6) (end 83.21 55.58) (width 0.4) (layer B.Cu) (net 8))
 (segment (start 83.65 55.58) (end 83.21 55.58) (width 0.4) (layer B.Cu) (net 8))
 (segment (start 84.4 56.33) (end 83.65 55.58) (width 0.4) (layer B.Cu) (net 8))
 (segment (start 84.4 56.8) (end 84.4 56.33) (width 0.4) (layer B.Cu) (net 8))
 (segment (start 84.1 57.1) (end 84.4 56.8) (width 0.4) (layer F.Cu) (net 8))
 (segment (start 81.55 57.1) (end 84.1 57.1) (width 0.4) (layer F.Cu) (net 8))
 (segment (start 74.12 57.1) (end 78.45 57.1) (width 0.4) (layer F.Cu) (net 10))
 (segment (start 73.3 56.28) (end 74.12 57.1) (width 0.4) (layer F.Cu) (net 10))
 (segment (start 73.3 51.2) (end 75.2 51.2) (width 0.4) (layer F.Cu) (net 12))
 (segment (start 75.2 51.2) (end 76 50.4) (width 0.4) (layer F.Cu) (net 12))
 (segment (start 76 50.4) (end 78.45 50.4) (width 0.4) (layer F.Cu) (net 12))
 (segment (start 73.3 58.82) (end 75.22 58.82) (width 0.4) (layer F.Cu) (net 9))
 (segment (start 75.22 58.82) (end 76 59.6) (width 0.4) (layer F.Cu) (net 9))
 (segment (start 76 59.6) (end 78.45 59.6) (width 0.4) (layer F.Cu) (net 9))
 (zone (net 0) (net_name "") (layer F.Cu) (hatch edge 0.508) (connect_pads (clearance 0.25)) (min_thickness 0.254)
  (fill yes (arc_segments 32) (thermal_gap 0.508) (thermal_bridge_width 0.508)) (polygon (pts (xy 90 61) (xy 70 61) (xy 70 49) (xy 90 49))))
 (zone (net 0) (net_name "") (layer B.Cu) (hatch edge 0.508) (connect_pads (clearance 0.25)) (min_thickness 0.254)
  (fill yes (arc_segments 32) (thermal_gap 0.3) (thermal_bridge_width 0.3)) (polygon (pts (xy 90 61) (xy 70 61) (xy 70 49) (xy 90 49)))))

